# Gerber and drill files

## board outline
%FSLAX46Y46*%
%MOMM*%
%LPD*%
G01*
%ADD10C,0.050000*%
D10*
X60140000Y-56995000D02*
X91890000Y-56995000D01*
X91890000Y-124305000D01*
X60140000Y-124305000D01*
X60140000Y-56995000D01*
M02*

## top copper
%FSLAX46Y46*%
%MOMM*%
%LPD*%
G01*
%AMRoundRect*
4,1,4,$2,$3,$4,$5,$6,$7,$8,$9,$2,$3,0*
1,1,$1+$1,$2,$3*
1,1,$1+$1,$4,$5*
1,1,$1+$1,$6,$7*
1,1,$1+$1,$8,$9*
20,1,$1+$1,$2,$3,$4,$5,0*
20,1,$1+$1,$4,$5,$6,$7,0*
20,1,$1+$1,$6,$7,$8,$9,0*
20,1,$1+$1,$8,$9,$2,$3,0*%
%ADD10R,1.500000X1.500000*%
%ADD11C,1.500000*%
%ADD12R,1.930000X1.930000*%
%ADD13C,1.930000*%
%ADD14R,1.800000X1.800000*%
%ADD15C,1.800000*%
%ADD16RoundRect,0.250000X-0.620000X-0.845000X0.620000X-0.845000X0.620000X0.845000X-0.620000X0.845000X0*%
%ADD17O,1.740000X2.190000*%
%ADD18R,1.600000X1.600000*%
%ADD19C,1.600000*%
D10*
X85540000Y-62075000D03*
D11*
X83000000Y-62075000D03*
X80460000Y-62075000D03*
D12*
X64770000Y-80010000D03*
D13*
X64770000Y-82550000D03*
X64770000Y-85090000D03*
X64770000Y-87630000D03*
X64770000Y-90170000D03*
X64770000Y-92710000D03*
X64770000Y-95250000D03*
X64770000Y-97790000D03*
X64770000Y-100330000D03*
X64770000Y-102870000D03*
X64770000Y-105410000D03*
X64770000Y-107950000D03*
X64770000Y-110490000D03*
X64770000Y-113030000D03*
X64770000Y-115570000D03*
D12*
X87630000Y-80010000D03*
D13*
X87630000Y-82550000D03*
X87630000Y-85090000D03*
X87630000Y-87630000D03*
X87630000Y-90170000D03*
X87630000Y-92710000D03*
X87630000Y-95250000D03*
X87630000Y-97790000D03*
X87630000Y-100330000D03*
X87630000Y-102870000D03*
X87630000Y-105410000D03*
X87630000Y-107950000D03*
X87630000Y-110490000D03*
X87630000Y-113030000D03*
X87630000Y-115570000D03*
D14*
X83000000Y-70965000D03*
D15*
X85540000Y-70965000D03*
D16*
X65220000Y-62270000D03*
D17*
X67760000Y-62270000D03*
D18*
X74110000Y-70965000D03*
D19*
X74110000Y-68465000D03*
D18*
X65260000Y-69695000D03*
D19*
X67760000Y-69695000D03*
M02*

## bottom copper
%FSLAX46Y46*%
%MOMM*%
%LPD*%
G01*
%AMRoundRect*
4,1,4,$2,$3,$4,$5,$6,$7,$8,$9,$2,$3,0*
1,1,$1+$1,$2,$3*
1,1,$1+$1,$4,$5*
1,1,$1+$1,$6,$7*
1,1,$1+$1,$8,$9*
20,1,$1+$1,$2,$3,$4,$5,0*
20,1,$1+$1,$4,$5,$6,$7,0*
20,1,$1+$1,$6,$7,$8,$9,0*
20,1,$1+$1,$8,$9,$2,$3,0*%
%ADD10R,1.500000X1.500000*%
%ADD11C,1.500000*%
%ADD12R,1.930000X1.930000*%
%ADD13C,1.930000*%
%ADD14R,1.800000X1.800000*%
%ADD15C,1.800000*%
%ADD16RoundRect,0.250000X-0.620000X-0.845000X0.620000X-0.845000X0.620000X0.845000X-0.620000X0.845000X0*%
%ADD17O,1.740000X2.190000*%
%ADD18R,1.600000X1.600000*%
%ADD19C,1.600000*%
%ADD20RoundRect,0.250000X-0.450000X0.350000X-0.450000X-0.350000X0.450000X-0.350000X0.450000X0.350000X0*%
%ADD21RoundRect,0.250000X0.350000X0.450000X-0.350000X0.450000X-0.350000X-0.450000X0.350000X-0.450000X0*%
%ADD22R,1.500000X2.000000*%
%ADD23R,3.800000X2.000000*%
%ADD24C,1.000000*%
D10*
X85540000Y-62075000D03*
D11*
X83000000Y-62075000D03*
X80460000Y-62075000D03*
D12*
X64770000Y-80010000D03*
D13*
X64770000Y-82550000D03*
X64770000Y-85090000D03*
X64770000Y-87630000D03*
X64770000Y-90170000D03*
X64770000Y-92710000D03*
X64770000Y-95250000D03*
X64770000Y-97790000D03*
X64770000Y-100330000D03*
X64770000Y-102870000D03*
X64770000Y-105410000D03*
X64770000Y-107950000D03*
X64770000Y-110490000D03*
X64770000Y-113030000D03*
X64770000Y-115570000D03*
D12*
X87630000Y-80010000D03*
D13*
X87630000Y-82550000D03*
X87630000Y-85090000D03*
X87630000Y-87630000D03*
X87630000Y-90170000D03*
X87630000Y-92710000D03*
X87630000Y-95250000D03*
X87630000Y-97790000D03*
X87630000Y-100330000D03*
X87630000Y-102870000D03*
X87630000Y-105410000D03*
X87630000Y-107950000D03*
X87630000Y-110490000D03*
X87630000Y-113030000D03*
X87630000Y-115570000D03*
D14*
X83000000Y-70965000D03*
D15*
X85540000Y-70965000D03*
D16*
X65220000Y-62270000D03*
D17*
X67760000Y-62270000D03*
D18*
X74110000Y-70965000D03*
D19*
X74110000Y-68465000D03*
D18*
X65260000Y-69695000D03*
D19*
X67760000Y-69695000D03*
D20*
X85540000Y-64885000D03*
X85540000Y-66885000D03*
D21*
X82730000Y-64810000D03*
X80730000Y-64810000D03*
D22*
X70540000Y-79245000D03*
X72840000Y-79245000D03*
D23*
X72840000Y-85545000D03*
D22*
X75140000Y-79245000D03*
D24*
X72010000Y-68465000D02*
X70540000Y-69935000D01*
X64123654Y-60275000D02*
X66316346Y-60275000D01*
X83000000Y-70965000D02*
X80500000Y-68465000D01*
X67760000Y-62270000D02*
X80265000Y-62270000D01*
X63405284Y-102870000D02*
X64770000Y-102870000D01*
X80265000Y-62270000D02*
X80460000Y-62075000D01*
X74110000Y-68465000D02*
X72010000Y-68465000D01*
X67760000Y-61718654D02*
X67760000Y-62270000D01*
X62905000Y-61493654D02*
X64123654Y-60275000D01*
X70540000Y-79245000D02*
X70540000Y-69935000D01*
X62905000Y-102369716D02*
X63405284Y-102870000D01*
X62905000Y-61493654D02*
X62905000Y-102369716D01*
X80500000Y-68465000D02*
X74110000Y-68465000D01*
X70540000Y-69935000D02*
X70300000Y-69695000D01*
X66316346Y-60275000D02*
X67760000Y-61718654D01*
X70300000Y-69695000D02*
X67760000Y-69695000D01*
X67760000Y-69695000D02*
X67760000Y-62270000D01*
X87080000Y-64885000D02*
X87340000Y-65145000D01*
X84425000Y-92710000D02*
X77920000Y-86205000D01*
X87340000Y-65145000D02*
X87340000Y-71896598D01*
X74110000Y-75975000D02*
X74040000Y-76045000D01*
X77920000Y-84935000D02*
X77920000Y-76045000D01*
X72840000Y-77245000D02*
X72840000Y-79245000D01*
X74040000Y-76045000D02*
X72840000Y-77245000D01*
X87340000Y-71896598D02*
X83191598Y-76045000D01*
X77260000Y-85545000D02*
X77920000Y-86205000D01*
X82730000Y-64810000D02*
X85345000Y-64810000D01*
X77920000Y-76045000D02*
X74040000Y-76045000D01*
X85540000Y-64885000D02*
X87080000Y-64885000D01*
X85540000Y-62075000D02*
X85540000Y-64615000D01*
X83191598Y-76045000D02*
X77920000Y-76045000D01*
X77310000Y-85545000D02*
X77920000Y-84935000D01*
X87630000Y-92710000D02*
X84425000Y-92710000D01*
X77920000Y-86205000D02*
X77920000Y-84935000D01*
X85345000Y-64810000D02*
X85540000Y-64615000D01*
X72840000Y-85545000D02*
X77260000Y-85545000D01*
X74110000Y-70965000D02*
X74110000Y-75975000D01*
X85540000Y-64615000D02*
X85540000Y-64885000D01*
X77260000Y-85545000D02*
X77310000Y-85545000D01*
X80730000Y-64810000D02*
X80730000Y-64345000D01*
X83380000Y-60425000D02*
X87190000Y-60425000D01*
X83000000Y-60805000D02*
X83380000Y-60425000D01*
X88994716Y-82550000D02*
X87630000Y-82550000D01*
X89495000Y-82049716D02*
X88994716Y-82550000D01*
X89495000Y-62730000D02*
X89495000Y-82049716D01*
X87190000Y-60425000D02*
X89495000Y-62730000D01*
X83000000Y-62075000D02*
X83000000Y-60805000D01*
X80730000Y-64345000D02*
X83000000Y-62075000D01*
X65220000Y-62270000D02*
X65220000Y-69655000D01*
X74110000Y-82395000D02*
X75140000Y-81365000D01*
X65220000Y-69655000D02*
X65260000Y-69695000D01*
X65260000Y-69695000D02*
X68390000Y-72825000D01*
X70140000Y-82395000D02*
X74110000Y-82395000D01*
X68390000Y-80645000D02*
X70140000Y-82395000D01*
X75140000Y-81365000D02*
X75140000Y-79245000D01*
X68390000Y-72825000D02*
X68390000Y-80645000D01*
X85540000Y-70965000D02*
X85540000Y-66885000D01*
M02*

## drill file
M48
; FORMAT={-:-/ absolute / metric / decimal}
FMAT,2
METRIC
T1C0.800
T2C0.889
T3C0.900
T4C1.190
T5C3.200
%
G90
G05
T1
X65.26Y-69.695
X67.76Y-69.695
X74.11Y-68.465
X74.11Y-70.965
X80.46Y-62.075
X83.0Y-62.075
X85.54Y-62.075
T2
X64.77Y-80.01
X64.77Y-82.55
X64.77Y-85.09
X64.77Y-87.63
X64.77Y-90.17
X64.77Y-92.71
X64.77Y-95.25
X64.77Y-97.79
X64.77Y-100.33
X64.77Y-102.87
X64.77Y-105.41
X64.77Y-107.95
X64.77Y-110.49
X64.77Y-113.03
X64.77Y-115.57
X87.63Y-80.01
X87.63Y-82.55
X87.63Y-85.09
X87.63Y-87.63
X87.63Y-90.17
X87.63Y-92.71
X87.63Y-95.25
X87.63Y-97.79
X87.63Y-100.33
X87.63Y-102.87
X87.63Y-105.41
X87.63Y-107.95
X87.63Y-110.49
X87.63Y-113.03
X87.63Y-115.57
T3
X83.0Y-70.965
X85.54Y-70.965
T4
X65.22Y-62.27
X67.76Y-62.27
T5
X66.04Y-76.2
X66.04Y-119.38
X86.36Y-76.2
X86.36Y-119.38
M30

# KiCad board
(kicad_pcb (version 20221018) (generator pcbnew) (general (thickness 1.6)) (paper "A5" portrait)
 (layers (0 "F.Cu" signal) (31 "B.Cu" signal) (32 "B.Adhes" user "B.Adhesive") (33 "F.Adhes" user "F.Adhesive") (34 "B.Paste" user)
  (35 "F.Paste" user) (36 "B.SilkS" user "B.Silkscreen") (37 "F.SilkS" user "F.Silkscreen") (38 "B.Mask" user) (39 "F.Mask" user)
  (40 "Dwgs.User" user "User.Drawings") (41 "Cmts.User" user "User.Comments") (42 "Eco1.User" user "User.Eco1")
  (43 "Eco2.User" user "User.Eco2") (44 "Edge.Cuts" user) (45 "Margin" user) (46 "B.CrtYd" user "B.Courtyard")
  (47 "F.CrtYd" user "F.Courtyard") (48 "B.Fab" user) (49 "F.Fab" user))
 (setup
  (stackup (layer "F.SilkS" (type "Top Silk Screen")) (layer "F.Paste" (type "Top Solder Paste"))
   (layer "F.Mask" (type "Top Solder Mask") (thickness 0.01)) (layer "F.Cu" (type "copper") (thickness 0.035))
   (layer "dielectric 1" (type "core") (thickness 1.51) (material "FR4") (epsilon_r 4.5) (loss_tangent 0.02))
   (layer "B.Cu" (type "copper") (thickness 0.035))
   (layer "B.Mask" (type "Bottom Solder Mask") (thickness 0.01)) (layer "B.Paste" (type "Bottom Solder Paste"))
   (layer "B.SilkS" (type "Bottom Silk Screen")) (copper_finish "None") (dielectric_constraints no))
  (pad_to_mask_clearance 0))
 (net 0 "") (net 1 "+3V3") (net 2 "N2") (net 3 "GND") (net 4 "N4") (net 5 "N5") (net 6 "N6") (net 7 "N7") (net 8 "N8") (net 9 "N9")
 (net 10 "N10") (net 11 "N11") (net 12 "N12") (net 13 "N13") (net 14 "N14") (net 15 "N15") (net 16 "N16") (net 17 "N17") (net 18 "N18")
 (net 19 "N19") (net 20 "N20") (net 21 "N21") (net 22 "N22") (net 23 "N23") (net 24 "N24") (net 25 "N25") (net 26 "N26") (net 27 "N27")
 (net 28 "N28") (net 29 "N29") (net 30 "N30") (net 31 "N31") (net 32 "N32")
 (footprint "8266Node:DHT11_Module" (layer "F.Cu") (at 85.54 62.075 -90)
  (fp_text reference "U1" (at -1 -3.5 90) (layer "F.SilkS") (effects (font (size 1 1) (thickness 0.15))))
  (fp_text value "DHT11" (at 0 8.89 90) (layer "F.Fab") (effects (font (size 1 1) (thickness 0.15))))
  (pad "1" thru_hole rect (at 0 0 270) (size 1.5 1.5) (drill 0.8) (layers "*.Cu" "*.Mask") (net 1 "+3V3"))
  (pad "2" thru_hole circle (at 0 2.54 270) (size 1.5 1.5) (drill 0.8) (layers "*.Cu" "*.Mask") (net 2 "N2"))
  (pad "3" thru_hole circle (at 0 5.08 270) (size 1.5 1.5) (drill 0.8) (layers "*.Cu" "*.Mask") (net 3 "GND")))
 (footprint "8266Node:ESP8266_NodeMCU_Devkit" (layer "F.Cu") (at 76.2 97.79)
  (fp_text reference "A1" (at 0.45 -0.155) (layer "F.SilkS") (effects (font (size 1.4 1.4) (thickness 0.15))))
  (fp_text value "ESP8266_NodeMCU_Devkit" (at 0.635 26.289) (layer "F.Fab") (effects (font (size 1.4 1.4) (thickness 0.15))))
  (pad "" np_thru_hole circle (at -10.16 -21.59) (size 3.2 3.2) (drill 3.2) (layers "*.Cu" "*.Mask"))
  (pad "" np_thru_hole circle (at -10.16 21.59) (size 3.2 3.2) (drill 3.2) (layers "*.Cu" "*.Mask"))
  (pad "" np_thru_hole circle (at 10.16 -21.59) (size 3.2 3.2) (drill 3.2) (layers "*.Cu" "*.Mask"))
  (pad "" np_thru_hole circle (at 10.16 21.59) (size 3.2 3.2) (drill 3.2) (layers "*.Cu" "*.Mask"))
  (pad "J1_1" thru_hole rect (at -11.43 -17.78) (size 1.93 1.93) (drill 0.889) (layers "*.Cu" "*.Mask") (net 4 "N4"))
  (pad "J1_2" thru_hole circle (at -11.43 -15.24) (size 1.93 1.93) (drill 0.889) (layers "*.Cu" "*.Mask") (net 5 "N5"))
  (pad "J1_3" thru_hole circle (at -11.43 -12.7) (size 1.93 1.93) (drill 0.889) (layers "*.Cu" "*.Mask") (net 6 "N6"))
  (pad "J1_4" thru_hole circle (at -11.43 -10.16) (size 1.93 1.93) (drill 0.889) (layers "*.Cu" "*.Mask") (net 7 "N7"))
  (pad "J1_5" thru_hole circle (at -11.43 -7.62) (size 1.93 1.93) (drill 0.889) (layers "*.Cu" "*.Mask") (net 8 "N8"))
  (pad "J1_6" thru_hole circle (at -11.43 -5.08) (size 1.93 1.93) (drill 0.889) (layers "*.Cu" "*.Mask") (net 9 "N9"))
  (pad "J1_7" thru_hole circle (at -11.43 -2.54) (size 1.93 1.93) (drill 0.889) (layers "*.Cu" "*.Mask") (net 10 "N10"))
  (pad "J1_8" thru_hole circle (at -11.43 0) (size 1.93 1.93) (drill 0.889) (layers "*.Cu" "*.Mask") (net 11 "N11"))
  (pad "J1_9" thru_hole circle (at -11.43 2.54) (size 1.93 1.93) (drill 0.889) (layers "*.Cu" "*.Mask") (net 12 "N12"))
  (pad "J1_10" thru_hole circle (at -11.43 5.08) (size 1.93 1.93) (drill 0.889) (layers "*.Cu" "*.Mask") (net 3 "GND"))
  (pad "J1_11" thru_hole circle (at -11.43 7.62) (size 1.93 1.93) (drill 0.889) (layers "*.Cu" "*.Mask") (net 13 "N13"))
  (pad "J1_12" thru_hole circle (at -11.43 10.16) (size 1.93 1.93) (drill 0.889) (layers "*.Cu" "*.Mask") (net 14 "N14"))
  (pad "J1_13" thru_hole circle (at -11.43 12.7) (size 1.93 1.93) (drill 0.889) (layers "*.Cu" "*.Mask") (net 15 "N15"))
  (pad "J1_14" thru_hole circle (at -11.43 15.24) (size 1.93 1.93) (drill 0.889) (layers "*.Cu" "*.Mask") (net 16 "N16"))
  (pad "J1_15" thru_hole circle (at -11.43 17.78) (size 1.93 1.93) (drill 0.889) (layers "*.Cu" "*.Mask") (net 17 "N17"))
  (pad "J2_1" thru_hole rect (at 11.43 -17.78) (size 1.93 1.93) (drill 0.889) (layers "*.Cu" "*.Mask") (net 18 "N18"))
  (pad "J2_2" thru_hole circle (at 11.43 -15.24) (size 1.93 1.93) (drill 0.889) (layers "*.Cu" "*.Mask") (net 2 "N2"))
  (pad "J2_3" thru_hole circle (at 11.43 -12.7) (size 1.93 1.93) (drill 0.889) (layers "*.Cu" "*.Mask") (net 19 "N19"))
  (pad "J2_4" thru_hole circle (at 11.43 -10.16) (size 1.93 1.93) (drill 0.889) (layers "*.Cu" "*.Mask") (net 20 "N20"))
  (pad "J2_5" thru_hole circle (at 11.43 -7.62) (size 1.93 1.93) (drill 0.889) (layers "*.Cu" "*.Mask") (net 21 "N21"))
  (pad "J2_6" thru_hole circle (at 11.43 -5.08) (size 1.93 1.93) (drill 0.889) (layers "*.Cu" "*.Mask") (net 1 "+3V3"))
  (pad "J2_7" thru_hole circle (at 11.43 -2.54) (size 1.93 1.93) (drill 0.889) (layers "*.Cu" "*.Mask") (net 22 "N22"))
  (pad "J2_8" thru_hole circle (at 11.43 0) (size 1.93 1.93) (drill 0.889) (layers "*.Cu" "*.Mask") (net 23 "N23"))
  (pad "J2_9" thru_hole circle (at 11.43 2.54) (size 1.93 1.93) (drill 0.889) (layers "*.Cu" "*.Mask") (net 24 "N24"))
  (pad "J2_10" thru_hole circle (at 11.43 5.08) (size 1.93 1.93) (drill 0.889) (layers "*.Cu" "*.Mask") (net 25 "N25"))
  (pad "J2_11" thru_hole circle (at 11.43 7.62) (size 1.93 1.93) (drill 0.889) (layers "*.Cu" "*.Mask") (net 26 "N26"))
  (pad "J2_12" thru_hole circle (at 11.43 10.16) (size 1.93 1.93) (drill 0.889) (layers "*.Cu" "*.Mask") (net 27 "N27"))
  (pad "J2_13" thru_hole circle (at 11.43 12.7) (size 1.93 1.93) (drill 0.889) (layers "*.Cu" "*.Mask") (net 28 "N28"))
  (pad "J2_14" thru_hole circle (at 11.43 15.24) (size 1.93 1.93) (drill 0.889) (layers "*.Cu" "*.Mask") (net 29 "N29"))
  (pad "J2_15" thru_hole circle (at 11.43 17.78) (size 1.93 1.93) (drill 0.889) (layers "*.Cu" "*.Mask") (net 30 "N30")))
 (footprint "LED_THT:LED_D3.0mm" (layer "F.Cu") (at 83 70.965)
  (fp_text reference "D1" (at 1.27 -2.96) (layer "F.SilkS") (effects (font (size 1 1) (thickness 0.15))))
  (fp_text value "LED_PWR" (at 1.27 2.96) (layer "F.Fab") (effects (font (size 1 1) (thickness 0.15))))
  (pad "1" thru_hole rect (at 0 0) (size 1.8 1.8) (drill 0.9) (layers "*.Cu" "*.Mask") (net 3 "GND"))
  (pad "2" thru_hole circle (at 2.54 0) (size 1.8 1.8) (drill 0.9) (layers "*.Cu" "*.Mask") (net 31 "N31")))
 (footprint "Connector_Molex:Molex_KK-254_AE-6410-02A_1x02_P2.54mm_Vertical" (layer "F.Cu") (at 65.22 62.27)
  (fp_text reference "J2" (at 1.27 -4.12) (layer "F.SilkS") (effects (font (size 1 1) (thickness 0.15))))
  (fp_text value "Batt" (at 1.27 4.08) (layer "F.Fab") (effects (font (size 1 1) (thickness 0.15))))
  (pad "1" thru_hole roundrect (at 0 0) (size 1.74 2.19) (drill 1.19) (layers "*.Cu" "*.Mask") (roundrect_rratio 0.1436781609)
   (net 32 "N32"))
  (pad "2" thru_hole oval (at 2.54 0) (size 1.74 2.19) (drill 1.19) (layers "*.Cu" "*.Mask") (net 3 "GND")))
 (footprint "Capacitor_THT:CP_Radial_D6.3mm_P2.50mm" (layer "F.Cu") (at 74.11 70.965 90)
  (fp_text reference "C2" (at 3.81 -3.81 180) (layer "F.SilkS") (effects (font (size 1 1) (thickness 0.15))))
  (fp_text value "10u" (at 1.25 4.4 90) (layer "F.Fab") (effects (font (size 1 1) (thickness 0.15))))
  (pad "1" thru_hole rect (at 0 0 90) (size 1.6 1.6) (drill 0.8) (layers "*.Cu" "*.Mask") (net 1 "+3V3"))
  (pad "2" thru_hole circle (at 2.5 0 90) (size 1.6 1.6) (drill 0.8) (layers "*.Cu" "*.Mask") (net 3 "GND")))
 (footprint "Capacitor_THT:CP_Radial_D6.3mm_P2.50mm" (layer "F.Cu") (at 65.26 69.695)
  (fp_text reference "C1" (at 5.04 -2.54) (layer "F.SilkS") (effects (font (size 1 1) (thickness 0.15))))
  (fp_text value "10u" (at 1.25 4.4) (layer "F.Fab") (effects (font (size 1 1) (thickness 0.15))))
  (pad "1" thru_hole rect (at 0 0) (size 1.6 1.6) (drill 0.8) (layers "*.Cu" "*.Mask") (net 32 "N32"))
  (pad "2" thru_hole circle (at 2.5 0) (size 1.6 1.6) (drill 0.8) (layers "*.Cu" "*.Mask") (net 3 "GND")))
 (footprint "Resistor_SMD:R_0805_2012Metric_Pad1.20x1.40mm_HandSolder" (layer "B.Cu") (at 85.54 65.885 -90)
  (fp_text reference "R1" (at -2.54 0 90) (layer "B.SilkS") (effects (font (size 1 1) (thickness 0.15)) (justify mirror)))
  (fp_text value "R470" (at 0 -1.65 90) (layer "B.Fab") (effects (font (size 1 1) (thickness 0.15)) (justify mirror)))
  (pad "1" smd roundrect (at -1 0 270) (size 1.2 1.4) (layers "B.Cu" "B.Paste" "B.Mask") (roundrect_rratio 0.2083333333) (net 1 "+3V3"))
  (pad "2" smd roundrect (at 1 0 270) (size 1.2 1.4) (layers "B.Cu" "B.Paste" "B.Mask") (roundrect_rratio 0.2083333333) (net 31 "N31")))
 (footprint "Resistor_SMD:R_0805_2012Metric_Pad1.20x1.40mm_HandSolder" (layer "B.Cu") (at 81.73 64.81 180)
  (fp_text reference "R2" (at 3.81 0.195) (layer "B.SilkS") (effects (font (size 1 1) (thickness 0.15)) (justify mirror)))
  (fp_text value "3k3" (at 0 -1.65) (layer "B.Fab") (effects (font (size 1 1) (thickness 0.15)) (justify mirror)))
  (pad "1" smd roundrect (at -1 0 180) (size 1.2 1.4) (layers "B.Cu" "B.Paste" "B.Mask") (roundrect_rratio 0.2083333333) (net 1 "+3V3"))
  (pad "2" smd roundrect (at 1 0 180) (size 1.2 1.4) (layers "B.Cu" "B.Paste" "B.Mask") (roundrect_rratio 0.2083333333) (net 2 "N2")))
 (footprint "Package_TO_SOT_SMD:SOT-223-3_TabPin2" (layer "B.Cu") (at 72.84 82.395 -90)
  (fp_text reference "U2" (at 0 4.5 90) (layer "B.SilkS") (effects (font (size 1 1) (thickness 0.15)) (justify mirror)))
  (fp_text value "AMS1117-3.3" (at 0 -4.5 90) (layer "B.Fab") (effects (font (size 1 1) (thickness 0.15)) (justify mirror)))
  (pad "1" smd rect (at -3.15 2.3 270) (size 2 1.5) (layers "B.Cu" "B.Paste" "B.Mask") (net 3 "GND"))
  (pad "2" smd rect (at -3.15 0 270) (size 2 1.5) (layers "B.Cu" "B.Paste" "B.Mask") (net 1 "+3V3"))
  (pad "2" smd rect (at 3.15 0 270) (size 2 3.8) (layers "B.Cu" "B.Paste" "B.Mask") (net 1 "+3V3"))
  (pad "3" smd rect (at -3.15 -2.3 270) (size 2 1.5) (layers "B.Cu" "B.Paste" "B.Mask") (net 32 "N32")))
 (gr_rect (start 60.14 56.995) (end 91.89 124.305) (stroke (width 0.05) (type default)) (fill none) (layer "Edge.Cuts"))
 (segment (start 72.01 68.465) (end 70.54 69.935) (width 1) (layer "B.Cu") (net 3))
 (segment (start 64.123654 60.275) (end 66.316346 60.275) (width 1) (layer "B.Cu") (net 3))
 (segment (start 83 70.965) (end 80.5 68.465) (width 1) (layer "B.Cu") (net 3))
 (segment (start 67.76 62.27) (end 80.265 62.27) (width 1) (layer "B.Cu") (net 3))
 (segment (start 63.405284 102.87) (end 64.77 102.87) (width 1) (layer "B.Cu") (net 3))
 (segment (start 80.265 62.27) (end 80.46 62.075) (width 1) (layer "B.Cu") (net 3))
 (segment (start 74.11 68.465) (end 72.01 68.465) (width 1) (layer "B.Cu") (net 3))
 (segment (start 67.76 61.718654) (end 67.76 62.27) (width 1) (layer "B.Cu") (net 3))
 (segment (start 62.905 61.493654) (end 64.123654 60.275) (width 1) (layer "B.Cu") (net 3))
 (segment (start 70.54 79.245) (end 70.54 69.935) (width 1) (layer "B.Cu") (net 3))
 (segment (start 62.905 102.369716) (end 63.405284 102.87) (width 1) (layer "B.Cu") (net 3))
 (segment (start 62.905 61.493654) (end 62.905 102.369716) (width 1) (layer "B.Cu") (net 3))
 (segment (start 80.5 68.465) (end 74.11 68.465) (width 1) (layer "B.Cu") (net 3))
 (segment (start 70.54 69.935) (end 70.3 69.695) (width 1) (layer "B.Cu") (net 3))
 (segment (start 66.316346 60.275) (end 67.76 61.718654) (width 1) (layer "B.Cu") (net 3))
 (segment (start 70.3 69.695) (end 67.76 69.695) (width 1) (layer "B.Cu") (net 3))
 (segment (start 67.76 69.695) (end 67.76 62.27) (width 1) (layer "B.Cu") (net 3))
 (segment (start 87.08 64.885) (end 87.34 65.145) (width 1) (layer "B.Cu") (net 1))
 (segment (start 84.425 92.71) (end 77.92 86.205) (width 1) (layer "B.Cu") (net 1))
 (segment (start 87.34 65.145) (end 87.34 71.896598) (width 1) (layer "B.Cu") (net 1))
 (segment (start 74.11 75.975) (end 74.04 76.045) (width 1) (layer "B.Cu") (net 1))
 (segment (start 77.92 84.935) (end 77.92 76.045) (width 1) (layer "B.Cu") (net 1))
 (segment (start 72.84 77.245) (end 72.84 79.245) (width 1) (layer "B.Cu") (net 1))
 (segment (start 74.04 76.045) (end 72.84 77.245) (width 1) (layer "B.Cu") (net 1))
 (segment (start 87.34 71.896598) (end 83.191598 76.045) (width 1) (layer "B.Cu") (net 1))
 (segment (start 77.26 85.545) (end 77.92 86.205) (width 1) (layer "B.Cu") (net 1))
 (segment (start 82.73 64.81) (end 85.345 64.81) (width 1) (layer "B.Cu") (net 1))
 (segment (start 77.92 76.045) (end 74.04 76.045) (width 1) (layer "B.Cu") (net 1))
 (segment (start 85.54 64.885) (end 87.08 64.885) (width 1) (layer "B.Cu") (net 1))
 (segment (start 85.54 62.075) (end 85.54 64.615) (width 1) (layer "B.Cu") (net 1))
 (segment (start 83.191598 76.045) (end 77.92 76.045) (width 1) (layer "B.Cu") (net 1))
 (segment (start 77.31 85.545) (end 77.92 84.935) (width 1) (layer "B.Cu") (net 1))
 (segment (start 87.63 92.71) (end 84.425 92.71) (width 1) (layer "B.Cu") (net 1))
 (segment (start 77.92 86.205) (end 77.92 84.935) (width 1) (layer "B.Cu") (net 1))
 (segment (start 85.345 64.81) (end 85.54 64.615) (width 1) (layer "B.Cu") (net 1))
 (segment (start 72.84 85.545) (end 77.26 85.545) (width 1) (layer "B.Cu") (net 1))
 (segment (start 74.11 70.965) (end 74.11 75.975) (width 1) (layer "B.Cu") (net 1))
 (segment (start 85.54 64.615) (end 85.54 64.885) (width 1) (layer "B.Cu") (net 1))
 (segment (start 77.26 85.545) (end 77.31 85.545) (width 1) (layer "B.Cu") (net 1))
 (segment (start 80.73 64.81) (end 80.73 64.345) (width 1) (layer "B.Cu") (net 2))
 (segment (start 83.38 60.425) (end 87.19 60.425) (width 1) (layer "B.Cu") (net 2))
 (segment (start 83 60.805) (end 83.38 60.425) (width 1) (layer "B.Cu") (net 2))
 (segment (start 88.994716 82.55) (end 87.63 82.55) (width 1) (layer "B.Cu") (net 2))
 (segment (start 89.495 82.049716) (end 88.994716 82.55) (width 1) (layer "B.Cu") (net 2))
 (segment (start 89.495 62.73) (end 89.495 82.049716) (width 1) (layer "B.Cu") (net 2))
 (segment (start 87.19 60.425) (end 89.495 62.73) (width 1) (layer "B.Cu") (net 2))
 (segment (start 83 62.075) (end 83 60.805) (width 1) (layer "B.Cu") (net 2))
 (segment (start 80.73 64.345) (end 83 62.075) (width 1) (layer "B.Cu") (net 2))
 (segment (start 65.22 62.27) (end 65.22 69.655) (width 1) (layer "B.Cu") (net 32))
 (segment (start 74.11 82.395) (end 75.14 81.365) (width 1) (layer "B.Cu") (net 32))
 (segment (start 65.22 69.655) (end 65.26 69.695) (width 1) (layer "B.Cu") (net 32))
 (segment (start 65.26 69.695) (end 68.39 72.825) (width 1) (layer "B.Cu") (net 32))
 (segment (start 70.14 82.395) (end 74.11 82.395) (width 1) (layer "B.Cu") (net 32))
 (segment (start 68.39 80.645) (end 70.14 82.395) (width 1) (layer "B.Cu") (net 32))
 (segment (start 75.14 81.365) (end 75.14 79.245) (width 1) (layer "B.Cu") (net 32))
 (segment (start 68.39 72.825) (end 68.39 80.645) (width 1) (layer "B.Cu") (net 32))
 (segment (start 85.54 70.965) (end 85.54 66.885) (width 1) (layer "B.Cu") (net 31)))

